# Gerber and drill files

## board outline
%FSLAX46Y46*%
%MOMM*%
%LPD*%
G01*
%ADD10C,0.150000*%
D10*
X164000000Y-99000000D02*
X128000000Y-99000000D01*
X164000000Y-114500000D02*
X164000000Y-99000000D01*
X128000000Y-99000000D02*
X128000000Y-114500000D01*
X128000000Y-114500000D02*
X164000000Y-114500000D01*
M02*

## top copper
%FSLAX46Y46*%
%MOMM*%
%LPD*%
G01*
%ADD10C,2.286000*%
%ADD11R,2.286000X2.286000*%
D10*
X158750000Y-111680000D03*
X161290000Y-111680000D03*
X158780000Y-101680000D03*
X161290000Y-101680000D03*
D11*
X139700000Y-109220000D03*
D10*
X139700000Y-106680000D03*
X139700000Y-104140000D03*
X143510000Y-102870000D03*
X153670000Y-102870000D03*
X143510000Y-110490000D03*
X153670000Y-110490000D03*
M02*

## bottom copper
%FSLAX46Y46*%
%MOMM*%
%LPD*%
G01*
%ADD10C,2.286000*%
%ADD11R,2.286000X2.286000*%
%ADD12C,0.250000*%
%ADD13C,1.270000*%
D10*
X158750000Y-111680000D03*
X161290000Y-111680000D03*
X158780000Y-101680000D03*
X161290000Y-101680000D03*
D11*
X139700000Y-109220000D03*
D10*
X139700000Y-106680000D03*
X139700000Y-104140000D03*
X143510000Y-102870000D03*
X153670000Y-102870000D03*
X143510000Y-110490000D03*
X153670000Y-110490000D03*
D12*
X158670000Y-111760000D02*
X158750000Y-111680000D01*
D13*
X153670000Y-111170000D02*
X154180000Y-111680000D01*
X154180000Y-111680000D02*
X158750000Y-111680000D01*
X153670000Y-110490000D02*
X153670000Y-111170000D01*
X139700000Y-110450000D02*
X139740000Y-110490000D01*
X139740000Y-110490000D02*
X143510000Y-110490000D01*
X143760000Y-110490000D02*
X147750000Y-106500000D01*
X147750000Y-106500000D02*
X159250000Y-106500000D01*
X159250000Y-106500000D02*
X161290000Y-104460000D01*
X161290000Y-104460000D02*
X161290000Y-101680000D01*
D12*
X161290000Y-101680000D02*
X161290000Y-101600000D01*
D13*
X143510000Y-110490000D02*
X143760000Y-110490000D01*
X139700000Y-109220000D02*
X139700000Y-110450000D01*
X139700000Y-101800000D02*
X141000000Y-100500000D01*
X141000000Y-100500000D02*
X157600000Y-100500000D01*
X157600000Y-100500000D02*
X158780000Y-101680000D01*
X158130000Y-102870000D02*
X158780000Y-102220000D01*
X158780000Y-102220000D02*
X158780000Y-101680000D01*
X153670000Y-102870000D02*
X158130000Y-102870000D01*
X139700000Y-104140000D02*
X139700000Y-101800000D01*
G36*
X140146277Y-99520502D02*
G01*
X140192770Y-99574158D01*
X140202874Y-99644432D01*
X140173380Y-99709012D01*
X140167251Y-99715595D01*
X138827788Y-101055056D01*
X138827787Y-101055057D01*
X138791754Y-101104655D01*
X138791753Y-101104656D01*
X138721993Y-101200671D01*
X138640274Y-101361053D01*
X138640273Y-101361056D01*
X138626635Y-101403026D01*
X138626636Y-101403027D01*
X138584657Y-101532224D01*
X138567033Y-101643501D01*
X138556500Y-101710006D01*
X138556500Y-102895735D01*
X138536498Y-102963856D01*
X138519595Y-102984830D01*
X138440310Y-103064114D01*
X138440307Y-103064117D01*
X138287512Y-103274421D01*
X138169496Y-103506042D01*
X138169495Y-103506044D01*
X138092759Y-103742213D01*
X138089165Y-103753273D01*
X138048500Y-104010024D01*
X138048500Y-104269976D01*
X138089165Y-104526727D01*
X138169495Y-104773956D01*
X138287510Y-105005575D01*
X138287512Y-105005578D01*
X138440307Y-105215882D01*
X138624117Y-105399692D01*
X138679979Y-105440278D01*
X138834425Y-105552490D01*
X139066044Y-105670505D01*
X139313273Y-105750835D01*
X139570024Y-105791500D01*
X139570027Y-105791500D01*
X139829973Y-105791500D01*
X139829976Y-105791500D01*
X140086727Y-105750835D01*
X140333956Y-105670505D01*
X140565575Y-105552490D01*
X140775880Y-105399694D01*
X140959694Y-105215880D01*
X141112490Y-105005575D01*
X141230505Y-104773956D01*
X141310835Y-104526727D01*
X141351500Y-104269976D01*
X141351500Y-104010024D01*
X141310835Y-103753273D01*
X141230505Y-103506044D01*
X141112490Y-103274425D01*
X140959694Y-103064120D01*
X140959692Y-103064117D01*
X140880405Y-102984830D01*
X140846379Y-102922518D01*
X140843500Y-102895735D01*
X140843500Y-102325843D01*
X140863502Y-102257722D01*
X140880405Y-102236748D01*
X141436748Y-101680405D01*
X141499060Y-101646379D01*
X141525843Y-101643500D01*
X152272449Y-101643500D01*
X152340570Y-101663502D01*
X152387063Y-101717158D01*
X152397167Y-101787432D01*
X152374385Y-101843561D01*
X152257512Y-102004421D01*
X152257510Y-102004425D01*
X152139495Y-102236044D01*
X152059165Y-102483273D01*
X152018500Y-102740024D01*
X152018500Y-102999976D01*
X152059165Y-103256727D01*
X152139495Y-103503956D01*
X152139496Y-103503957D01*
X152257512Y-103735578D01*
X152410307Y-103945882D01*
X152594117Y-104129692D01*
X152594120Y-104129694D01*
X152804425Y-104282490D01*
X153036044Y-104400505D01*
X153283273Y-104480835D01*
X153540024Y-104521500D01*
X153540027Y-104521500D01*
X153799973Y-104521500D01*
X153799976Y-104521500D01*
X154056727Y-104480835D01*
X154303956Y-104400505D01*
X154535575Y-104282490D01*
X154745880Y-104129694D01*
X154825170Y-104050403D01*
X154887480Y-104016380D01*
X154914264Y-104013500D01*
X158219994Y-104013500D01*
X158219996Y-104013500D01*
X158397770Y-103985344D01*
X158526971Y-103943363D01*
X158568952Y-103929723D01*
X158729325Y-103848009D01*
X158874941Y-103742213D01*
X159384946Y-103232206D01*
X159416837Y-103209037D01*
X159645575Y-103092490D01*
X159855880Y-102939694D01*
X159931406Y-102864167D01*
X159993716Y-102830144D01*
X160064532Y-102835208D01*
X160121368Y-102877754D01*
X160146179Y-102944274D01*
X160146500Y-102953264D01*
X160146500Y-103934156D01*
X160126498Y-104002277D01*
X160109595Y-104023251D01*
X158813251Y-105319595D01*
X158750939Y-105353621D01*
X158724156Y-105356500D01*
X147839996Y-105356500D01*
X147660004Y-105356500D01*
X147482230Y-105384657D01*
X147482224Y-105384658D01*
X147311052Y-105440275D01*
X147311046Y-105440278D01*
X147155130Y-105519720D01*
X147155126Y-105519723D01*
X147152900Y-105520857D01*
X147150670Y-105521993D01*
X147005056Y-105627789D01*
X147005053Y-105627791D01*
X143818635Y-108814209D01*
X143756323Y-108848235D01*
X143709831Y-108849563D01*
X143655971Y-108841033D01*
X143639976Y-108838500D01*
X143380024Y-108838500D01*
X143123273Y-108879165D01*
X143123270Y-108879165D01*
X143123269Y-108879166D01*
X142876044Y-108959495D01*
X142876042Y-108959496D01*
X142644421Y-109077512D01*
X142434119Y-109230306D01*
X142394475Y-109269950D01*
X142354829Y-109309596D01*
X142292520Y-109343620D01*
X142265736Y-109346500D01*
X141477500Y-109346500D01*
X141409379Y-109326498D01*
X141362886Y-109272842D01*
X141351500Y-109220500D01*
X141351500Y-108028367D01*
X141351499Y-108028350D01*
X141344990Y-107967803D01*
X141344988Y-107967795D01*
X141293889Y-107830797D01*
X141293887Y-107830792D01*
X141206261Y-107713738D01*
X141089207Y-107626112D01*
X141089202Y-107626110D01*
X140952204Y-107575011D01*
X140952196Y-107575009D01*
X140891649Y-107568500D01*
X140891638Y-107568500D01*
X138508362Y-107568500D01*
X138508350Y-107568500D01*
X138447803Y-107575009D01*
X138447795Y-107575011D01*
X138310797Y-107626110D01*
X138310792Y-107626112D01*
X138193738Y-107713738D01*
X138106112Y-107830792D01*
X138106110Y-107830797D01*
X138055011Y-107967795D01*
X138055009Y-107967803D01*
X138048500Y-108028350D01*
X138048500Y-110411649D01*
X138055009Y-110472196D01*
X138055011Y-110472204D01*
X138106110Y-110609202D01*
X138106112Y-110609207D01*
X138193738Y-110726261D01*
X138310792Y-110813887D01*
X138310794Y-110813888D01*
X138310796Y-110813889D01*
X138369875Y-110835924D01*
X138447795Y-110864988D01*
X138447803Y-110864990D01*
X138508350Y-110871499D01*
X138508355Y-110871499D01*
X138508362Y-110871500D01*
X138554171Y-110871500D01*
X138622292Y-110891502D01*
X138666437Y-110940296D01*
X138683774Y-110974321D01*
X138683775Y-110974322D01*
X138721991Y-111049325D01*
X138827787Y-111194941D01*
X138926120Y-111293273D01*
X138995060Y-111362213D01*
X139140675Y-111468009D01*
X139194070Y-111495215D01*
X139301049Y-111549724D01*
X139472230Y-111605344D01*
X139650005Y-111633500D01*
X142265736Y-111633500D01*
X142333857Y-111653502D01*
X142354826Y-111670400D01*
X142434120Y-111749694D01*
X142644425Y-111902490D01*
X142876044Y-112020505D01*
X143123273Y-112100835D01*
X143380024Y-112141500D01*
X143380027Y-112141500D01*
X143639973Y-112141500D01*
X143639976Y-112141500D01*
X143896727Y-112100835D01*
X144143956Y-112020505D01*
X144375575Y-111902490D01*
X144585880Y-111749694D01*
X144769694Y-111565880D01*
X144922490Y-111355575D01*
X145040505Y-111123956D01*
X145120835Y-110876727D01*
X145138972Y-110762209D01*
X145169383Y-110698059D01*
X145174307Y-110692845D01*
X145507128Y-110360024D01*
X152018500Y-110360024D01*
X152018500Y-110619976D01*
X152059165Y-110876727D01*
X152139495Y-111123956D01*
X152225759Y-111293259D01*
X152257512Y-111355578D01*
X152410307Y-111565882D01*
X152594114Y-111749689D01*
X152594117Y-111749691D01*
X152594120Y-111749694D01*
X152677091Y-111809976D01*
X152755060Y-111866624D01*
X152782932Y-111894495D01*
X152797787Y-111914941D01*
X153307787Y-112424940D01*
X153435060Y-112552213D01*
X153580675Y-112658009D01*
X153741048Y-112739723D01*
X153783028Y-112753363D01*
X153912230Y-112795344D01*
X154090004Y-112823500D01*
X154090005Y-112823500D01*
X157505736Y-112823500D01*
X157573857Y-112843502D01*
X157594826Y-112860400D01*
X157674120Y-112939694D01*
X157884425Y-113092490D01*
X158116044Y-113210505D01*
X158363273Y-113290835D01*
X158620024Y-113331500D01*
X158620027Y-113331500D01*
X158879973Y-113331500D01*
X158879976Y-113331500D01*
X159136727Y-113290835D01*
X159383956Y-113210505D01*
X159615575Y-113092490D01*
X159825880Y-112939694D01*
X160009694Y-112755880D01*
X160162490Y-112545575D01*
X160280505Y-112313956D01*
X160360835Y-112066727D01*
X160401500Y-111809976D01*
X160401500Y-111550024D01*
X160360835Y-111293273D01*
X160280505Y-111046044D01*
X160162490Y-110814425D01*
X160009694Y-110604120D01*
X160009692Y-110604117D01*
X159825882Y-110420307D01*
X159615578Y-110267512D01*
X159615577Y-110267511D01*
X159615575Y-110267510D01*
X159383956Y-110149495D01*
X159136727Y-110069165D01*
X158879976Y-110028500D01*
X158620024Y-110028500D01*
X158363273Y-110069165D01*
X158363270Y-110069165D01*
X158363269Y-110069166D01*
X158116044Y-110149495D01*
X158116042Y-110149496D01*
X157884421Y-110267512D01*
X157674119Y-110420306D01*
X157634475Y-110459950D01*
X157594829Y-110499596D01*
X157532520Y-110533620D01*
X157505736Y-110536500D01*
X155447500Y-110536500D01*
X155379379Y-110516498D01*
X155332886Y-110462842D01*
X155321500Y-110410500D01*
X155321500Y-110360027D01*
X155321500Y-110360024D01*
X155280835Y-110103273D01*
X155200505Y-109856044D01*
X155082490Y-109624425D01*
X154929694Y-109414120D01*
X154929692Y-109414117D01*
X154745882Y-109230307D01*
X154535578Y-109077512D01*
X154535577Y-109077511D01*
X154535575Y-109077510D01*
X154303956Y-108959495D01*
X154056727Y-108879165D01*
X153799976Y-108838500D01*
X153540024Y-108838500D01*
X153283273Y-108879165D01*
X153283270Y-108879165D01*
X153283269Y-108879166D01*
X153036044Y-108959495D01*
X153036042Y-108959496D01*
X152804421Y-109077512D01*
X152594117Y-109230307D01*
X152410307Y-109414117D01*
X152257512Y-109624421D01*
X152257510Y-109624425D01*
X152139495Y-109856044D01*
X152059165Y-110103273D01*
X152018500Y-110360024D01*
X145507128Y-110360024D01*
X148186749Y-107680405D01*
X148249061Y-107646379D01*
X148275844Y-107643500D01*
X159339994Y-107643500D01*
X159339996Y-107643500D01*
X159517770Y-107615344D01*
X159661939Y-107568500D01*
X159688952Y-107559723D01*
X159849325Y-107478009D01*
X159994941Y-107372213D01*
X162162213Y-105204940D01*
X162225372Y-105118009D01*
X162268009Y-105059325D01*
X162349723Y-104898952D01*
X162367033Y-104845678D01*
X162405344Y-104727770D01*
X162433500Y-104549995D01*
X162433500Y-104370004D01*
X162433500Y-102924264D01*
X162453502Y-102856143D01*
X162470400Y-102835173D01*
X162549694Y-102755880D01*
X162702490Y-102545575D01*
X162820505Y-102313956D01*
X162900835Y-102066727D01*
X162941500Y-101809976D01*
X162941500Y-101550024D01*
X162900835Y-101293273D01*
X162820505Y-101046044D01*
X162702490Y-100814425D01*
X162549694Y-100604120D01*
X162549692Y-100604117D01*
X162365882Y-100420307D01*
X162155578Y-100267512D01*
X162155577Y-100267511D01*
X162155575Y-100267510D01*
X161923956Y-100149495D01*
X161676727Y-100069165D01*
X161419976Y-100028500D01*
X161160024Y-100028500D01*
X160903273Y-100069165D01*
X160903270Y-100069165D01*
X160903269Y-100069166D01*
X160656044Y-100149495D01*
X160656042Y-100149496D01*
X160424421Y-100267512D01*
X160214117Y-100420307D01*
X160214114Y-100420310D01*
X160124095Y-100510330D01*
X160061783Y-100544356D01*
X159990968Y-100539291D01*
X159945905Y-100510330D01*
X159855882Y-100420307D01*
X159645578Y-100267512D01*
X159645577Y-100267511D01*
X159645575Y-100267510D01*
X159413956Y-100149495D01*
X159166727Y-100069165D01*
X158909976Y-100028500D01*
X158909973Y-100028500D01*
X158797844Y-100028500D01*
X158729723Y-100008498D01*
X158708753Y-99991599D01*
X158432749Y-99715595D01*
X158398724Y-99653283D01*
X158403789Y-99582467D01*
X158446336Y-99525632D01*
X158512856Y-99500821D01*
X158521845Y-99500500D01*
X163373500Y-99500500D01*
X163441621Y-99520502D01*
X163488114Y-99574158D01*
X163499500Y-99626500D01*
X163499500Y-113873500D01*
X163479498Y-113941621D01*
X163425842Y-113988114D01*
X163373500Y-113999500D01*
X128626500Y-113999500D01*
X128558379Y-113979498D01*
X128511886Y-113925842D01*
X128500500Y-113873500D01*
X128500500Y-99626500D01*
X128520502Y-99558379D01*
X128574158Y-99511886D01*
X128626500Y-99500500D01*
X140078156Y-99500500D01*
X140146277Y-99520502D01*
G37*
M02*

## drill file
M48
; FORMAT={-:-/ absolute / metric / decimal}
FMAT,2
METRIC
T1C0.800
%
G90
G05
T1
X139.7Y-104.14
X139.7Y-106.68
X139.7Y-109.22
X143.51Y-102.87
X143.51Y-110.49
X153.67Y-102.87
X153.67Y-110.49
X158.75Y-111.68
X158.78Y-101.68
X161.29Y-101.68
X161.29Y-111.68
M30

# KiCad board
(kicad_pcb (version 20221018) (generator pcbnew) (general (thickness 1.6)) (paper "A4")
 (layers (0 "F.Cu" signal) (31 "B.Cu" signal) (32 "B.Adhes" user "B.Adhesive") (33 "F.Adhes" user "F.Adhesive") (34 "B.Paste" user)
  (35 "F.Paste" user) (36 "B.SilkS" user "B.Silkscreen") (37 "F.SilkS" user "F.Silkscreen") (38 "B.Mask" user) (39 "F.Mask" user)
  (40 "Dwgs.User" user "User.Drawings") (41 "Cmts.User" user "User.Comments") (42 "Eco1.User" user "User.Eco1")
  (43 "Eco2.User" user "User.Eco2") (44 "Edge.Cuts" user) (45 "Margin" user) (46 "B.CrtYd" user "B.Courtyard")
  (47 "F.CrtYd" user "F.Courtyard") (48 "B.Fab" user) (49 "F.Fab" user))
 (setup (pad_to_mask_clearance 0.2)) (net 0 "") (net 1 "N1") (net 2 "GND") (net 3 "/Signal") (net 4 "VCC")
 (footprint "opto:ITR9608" (layer "F.Cu") (at 160.02 106.68 90)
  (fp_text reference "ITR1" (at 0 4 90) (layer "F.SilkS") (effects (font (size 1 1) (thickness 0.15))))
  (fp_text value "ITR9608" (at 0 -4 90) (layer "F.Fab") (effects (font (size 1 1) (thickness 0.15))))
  (pad "1" thru_hole circle (at -5 -1.27 90) (size 2.286 2.286) (drill 0.8) (layers "*.Cu" "*.Mask" "F.SilkS") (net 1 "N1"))
  (pad "2" thru_hole circle (at -5 1.27 90) (size 2.286 2.286) (drill 0.8) (layers "*.Cu" "*.Mask" "F.SilkS") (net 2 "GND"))
  (pad "3" thru_hole circle (at 5 -1.24 90) (size 2.286 2.286) (drill 0.8) (layers "*.Cu" "*.Mask" "F.SilkS") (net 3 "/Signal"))
  (pad "4" thru_hole circle (at 5 1.27 90) (size 2.286 2.286) (drill 0.8) (layers "*.Cu" "*.Mask" "F.SilkS") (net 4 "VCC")))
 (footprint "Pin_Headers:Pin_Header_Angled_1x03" (layer "F.Cu") (at 139.7 109.22 180)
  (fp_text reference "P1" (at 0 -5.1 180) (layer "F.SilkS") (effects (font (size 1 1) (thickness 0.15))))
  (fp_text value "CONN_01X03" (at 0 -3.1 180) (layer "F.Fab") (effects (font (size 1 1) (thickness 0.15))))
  (pad "1" thru_hole rect (at 0 0 180) (size 2.286 2.286) (drill 0.8) (layers "*.Cu" "*.Mask" "F.SilkS") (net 4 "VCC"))
  (pad "2" thru_hole circle (at 0 2.54 180) (size 2.286 2.286) (drill 0.8) (layers "*.Cu" "*.Mask" "F.SilkS") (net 2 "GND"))
  (pad "3" thru_hole circle (at 0 5.08 180) (size 2.286 2.286) (drill 0.8) (layers "*.Cu" "*.Mask" "F.SilkS") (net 3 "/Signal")))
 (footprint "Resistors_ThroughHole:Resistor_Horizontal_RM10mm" (layer "F.Cu") (at 148.59 102.87)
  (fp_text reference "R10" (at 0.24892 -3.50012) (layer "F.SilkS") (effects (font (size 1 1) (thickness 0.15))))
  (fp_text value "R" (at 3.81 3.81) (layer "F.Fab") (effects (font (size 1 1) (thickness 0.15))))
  (pad "1" thru_hole circle (at -5.08 0) (size 2.286 2.286) (drill 0.8) (layers "*.Cu" "*.SilkS" "*.Mask") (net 2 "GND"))
  (pad "2" thru_hole circle (at 5.08 0) (size 2.286 2.286) (drill 0.8) (layers "*.Cu" "*.SilkS" "*.Mask") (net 3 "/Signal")))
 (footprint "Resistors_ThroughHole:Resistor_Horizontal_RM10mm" (layer "F.Cu") (at 148.59 110.49)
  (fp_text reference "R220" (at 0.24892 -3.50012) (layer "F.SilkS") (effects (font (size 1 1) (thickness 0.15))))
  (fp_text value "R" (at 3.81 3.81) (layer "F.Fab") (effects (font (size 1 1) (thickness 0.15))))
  (pad "1" thru_hole circle (at -5.08 0) (size 2.286 2.286) (drill 0.8) (layers "*.Cu" "*.SilkS" "*.Mask") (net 4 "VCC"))
  (pad "2" thru_hole circle (at 5.08 0) (size 2.286 2.286) (drill 0.8) (layers "*.Cu" "*.SilkS" "*.Mask") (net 1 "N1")))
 (gr_line (start 164 99) (end 128 99) (stroke (width 0.15) (type solid)) (layer "Edge.Cuts"))
 (gr_line (start 164 114.5) (end 164 99) (stroke (width 0.15) (type solid)) (layer "Edge.Cuts"))
 (gr_line (start 128 99) (end 128 114.5) (stroke (width 0.15) (type solid)) (layer "Edge.Cuts"))
 (gr_line (start 128 114.5) (end 164 114.5) (stroke (width 0.15) (type solid)) (layer "Edge.Cuts"))
 (segment (start 158.67 111.76) (end 158.75 111.68) (width 0.25) (layer "B.Cu") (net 1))
 (segment (start 153.67 111.17) (end 154.18 111.68) (width 1.27) (layer "B.Cu") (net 1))
 (segment (start 154.18 111.68) (end 158.75 111.68) (width 1.27) (layer "B.Cu") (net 1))
 (segment (start 153.67 110.49) (end 153.67 111.17) (width 1.27) (layer "B.Cu") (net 1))
 (segment (start 139.7 110.45) (end 139.74 110.49) (width 1.27) (layer "B.Cu") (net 4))
 (segment (start 139.74 110.49) (end 143.51 110.49) (width 1.27) (layer "B.Cu") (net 4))
 (segment (start 143.76 110.49) (end 147.75 106.5) (width 1.27) (layer "B.Cu") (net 4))
 (segment (start 147.75 106.5) (end 159.25 106.5) (width 1.27) (layer "B.Cu") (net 4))
 (segment (start 159.25 106.5) (end 161.29 104.46) (width 1.27) (layer "B.Cu") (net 4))
 (segment (start 161.29 104.46) (end 161.29 101.68) (width 1.27) (layer "B.Cu") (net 4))
 (segment (start 161.29 101.68) (end 161.29 101.6) (width 0.25) (layer "B.Cu") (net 4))
 (segment (start 143.51 110.49) (end 143.76 110.49) (width 1.27) (layer "B.Cu") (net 4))
 (segment (start 139.7 109.22) (end 139.7 110.45) (width 1.27) (layer "B.Cu") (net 4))
 (segment (start 139.7 101.8) (end 141 100.5) (width 1.27) (layer "B.Cu") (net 3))
 (segment (start 141 100.5) (end 157.6 100.5) (width 1.27) (layer "B.Cu") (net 3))
 (segment (start 157.6 100.5) (end 158.78 101.68) (width 1.27) (layer "B.Cu") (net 3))
 (segment (start 158.13 102.87) (end 158.78 102.22) (width 1.27) (layer "B.Cu") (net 3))
 (segment (start 158.78 102.22) (end 158.78 101.68) (width 1.27) (layer "B.Cu") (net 3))
 (segment (start 153.67 102.87) (end 158.13 102.87) (width 1.27) (layer "B.Cu") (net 3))
 (segment (start 139.7 104.14) (end 139.7 101.8) (width 1.27) (layer "B.Cu") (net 3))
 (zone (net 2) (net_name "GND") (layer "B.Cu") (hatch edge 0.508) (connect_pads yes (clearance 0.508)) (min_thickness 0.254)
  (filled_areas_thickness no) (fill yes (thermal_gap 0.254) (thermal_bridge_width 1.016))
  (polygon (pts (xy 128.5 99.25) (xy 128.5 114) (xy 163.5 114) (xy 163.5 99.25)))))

